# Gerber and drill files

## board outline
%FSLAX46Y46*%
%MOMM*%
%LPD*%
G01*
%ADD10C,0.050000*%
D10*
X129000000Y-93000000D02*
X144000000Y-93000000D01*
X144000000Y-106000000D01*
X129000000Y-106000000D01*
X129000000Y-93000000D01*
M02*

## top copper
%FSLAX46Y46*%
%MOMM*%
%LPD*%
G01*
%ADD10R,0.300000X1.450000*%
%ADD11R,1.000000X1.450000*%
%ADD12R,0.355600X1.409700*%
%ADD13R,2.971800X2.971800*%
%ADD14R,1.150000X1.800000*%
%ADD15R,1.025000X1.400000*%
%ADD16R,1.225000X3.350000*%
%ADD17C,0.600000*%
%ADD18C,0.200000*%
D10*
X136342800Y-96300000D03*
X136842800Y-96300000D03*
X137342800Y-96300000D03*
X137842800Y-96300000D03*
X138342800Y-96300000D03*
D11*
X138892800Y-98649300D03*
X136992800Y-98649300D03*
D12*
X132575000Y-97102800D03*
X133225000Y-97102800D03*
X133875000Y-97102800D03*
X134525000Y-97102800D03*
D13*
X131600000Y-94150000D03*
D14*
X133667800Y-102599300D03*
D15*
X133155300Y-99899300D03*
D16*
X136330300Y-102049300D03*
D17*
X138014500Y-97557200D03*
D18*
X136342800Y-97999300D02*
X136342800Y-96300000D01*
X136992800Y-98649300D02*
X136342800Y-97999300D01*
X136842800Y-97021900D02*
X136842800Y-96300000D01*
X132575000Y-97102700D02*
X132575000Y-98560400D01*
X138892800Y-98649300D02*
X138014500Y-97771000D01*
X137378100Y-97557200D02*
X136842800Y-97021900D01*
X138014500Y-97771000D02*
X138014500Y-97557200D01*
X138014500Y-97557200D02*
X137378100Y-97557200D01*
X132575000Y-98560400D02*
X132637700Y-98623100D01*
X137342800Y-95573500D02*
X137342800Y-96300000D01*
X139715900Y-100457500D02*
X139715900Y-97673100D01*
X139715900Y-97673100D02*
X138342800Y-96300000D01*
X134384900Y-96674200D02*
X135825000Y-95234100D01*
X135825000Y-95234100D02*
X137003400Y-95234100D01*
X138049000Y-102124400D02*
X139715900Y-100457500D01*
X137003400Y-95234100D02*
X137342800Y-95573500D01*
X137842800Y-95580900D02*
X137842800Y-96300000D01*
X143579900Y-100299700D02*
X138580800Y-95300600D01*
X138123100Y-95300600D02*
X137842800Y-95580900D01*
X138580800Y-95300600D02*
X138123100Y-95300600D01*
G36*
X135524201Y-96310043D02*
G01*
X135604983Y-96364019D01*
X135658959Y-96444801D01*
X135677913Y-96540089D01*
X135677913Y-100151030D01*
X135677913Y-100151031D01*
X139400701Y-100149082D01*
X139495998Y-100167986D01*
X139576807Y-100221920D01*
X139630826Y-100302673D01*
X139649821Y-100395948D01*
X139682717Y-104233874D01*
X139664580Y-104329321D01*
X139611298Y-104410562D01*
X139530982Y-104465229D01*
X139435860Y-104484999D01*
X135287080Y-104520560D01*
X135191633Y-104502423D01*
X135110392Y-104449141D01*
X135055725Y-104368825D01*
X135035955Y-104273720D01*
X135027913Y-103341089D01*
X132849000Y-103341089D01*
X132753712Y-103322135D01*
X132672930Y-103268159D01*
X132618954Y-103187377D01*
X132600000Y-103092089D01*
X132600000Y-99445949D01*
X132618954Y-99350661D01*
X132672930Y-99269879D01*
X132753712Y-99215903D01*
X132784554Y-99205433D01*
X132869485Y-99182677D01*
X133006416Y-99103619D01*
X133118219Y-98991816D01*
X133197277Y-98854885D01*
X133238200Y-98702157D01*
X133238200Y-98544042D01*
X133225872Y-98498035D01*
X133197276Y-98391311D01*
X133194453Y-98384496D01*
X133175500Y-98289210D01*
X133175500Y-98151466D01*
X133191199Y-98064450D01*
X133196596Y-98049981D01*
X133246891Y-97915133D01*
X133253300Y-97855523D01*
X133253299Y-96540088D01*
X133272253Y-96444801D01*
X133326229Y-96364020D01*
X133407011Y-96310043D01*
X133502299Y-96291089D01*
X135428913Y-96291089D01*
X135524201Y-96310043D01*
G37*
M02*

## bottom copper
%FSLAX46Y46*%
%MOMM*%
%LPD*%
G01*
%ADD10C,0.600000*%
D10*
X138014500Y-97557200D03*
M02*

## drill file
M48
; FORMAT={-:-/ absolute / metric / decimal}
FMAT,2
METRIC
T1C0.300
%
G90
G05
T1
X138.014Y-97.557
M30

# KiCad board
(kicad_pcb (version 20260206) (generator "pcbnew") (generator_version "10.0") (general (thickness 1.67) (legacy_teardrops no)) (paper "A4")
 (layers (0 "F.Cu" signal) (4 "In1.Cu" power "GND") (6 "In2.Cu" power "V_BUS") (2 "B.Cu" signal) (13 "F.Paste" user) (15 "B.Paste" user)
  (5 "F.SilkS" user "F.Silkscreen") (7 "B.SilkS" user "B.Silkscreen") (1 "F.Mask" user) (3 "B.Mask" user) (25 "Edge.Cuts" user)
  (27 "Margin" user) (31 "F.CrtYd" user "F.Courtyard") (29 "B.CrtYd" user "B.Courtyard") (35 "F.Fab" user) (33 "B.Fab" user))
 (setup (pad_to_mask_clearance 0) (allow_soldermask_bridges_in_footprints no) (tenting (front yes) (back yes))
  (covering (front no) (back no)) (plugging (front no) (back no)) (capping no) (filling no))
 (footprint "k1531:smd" (layer "F.Cu") (at 136.3428 96.3)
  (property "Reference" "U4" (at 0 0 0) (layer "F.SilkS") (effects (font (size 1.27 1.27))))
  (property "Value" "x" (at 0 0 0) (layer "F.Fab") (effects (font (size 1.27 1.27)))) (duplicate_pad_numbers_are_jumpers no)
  (pad "1" smd rect (at 0 0) (size 0.3 1.45) (layers "F.Cu" "F.Mask") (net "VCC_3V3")))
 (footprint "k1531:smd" (layer "F.Cu") (at 136.8428 96.3)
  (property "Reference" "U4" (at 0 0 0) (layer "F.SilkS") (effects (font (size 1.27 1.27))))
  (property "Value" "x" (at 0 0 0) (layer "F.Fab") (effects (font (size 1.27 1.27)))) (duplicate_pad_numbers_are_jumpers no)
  (pad "1" smd rect (at 0 0) (size 0.3 1.45) (layers "F.Cu" "F.Mask") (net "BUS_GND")))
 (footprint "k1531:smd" (layer "F.Cu") (at 137.3428 96.3)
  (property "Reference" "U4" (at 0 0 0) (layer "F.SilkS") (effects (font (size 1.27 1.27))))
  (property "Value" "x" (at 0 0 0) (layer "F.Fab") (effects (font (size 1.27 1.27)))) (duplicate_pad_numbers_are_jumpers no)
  (pad "1" smd rect (at 0 0) (size 0.3 1.45) (layers "F.Cu" "F.Mask") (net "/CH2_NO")))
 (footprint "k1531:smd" (layer "F.Cu") (at 137.8428 96.3)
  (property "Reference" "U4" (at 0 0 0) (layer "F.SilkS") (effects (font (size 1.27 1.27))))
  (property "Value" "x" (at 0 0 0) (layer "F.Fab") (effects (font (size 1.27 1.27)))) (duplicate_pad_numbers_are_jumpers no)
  (pad "1" smd rect (at 0 0) (size 0.3 1.45) (layers "F.Cu" "F.Mask") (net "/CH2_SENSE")))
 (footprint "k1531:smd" (layer "F.Cu") (at 138.3428 96.3)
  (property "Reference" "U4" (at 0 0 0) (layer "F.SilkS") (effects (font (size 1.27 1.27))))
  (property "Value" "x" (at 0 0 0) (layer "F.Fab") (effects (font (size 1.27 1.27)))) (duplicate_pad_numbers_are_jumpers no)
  (pad "1" smd rect (at 0 0) (size 0.3 1.45) (layers "F.Cu" "F.Mask") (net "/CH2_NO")))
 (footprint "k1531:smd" (layer "F.Cu") (at 138.8928 98.6493)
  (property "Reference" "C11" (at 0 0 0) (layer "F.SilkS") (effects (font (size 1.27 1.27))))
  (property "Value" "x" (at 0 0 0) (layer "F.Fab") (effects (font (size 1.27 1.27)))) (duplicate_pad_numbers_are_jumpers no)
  (pad "1" smd rect (at 0 0) (size 1 1.45) (layers "F.Cu" "F.Mask") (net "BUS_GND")))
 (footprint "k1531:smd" (layer "F.Cu") (at 136.9928 98.6493)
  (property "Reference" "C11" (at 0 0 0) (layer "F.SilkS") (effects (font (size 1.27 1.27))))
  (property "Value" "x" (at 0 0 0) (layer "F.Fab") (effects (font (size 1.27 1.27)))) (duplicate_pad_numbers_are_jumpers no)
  (pad "1" smd rect (at 0 0) (size 1 1.45) (layers "F.Cu" "F.Mask") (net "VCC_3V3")))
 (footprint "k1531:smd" (layer "F.Cu") (at 132.575 97.1028)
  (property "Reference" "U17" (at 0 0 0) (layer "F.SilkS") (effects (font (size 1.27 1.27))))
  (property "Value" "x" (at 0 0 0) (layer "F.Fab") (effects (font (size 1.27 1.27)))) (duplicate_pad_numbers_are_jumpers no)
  (pad "1" smd rect (at 0 0) (size 0.3556 1.4097) (layers "F.Cu" "F.Mask") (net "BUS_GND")))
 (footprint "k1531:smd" (layer "F.Cu") (at 133.225 97.1028)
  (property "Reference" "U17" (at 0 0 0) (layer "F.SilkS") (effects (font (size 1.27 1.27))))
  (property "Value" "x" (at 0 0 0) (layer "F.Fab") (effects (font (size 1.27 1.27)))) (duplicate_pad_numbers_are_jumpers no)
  (pad "1" smd rect (at 0 0) (size 0.3556 1.4097) (layers "F.Cu" "F.Mask") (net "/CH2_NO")))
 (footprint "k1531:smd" (layer "F.Cu") (at 133.875 97.1028)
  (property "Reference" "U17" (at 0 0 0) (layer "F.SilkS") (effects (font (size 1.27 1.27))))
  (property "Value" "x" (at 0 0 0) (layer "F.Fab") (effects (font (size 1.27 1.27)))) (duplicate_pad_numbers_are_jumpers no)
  (pad "1" smd rect (at 0 0) (size 0.3556 1.4097) (layers "F.Cu" "F.Mask") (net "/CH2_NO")))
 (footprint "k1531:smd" (layer "F.Cu") (at 134.525 97.1028)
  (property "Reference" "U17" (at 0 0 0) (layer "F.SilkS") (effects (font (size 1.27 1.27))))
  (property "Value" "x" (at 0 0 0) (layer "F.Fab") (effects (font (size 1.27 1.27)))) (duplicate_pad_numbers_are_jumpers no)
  (pad "1" smd rect (at 0 0) (size 0.3556 1.4097) (layers "F.Cu" "F.Mask") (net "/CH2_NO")))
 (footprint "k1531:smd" (layer "F.Cu") (at 131.6 94.15)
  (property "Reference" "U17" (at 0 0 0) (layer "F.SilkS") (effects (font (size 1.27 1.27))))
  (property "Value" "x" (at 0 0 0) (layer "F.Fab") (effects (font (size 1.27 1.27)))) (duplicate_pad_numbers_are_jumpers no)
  (pad "1" smd rect (at 0 0) (size 2.9718 2.9718) (layers "F.Cu" "F.Mask") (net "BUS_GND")))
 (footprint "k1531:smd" (layer "F.Cu") (at 133.6678 102.5993)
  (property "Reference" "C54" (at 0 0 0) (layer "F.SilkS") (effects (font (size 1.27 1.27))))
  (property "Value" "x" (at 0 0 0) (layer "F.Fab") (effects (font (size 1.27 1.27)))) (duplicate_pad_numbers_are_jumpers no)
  (pad "1" smd rect (at 0 0) (size 1.15 1.8) (layers "F.Cu" "F.Mask") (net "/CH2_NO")))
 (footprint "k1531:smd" (layer "F.Cu") (at 133.1553 99.8993)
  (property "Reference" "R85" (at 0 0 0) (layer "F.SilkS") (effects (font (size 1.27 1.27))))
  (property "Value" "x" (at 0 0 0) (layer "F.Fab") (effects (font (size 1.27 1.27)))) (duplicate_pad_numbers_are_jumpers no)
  (pad "1" smd rect (at 0 0) (size 1.025 1.4) (layers "F.Cu" "F.Mask") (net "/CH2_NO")))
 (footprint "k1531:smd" (layer "F.Cu") (at 136.3303 102.0493)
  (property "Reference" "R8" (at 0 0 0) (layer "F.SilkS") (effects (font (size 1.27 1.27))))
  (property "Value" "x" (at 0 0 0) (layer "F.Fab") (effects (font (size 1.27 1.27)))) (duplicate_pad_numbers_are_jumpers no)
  (pad "1" smd rect (at 0 0) (size 1.225 3.35) (layers "F.Cu" "F.Mask") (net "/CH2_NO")))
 (gr_rect (start 129 93) (end 144 106) (stroke (width 0.05) (type default)) (fill no) (layer "Edge.Cuts"))
 (segment (start 136.3428 97.9993) (end 136.3428 96.3) (width 0.2) (layer "F.Cu") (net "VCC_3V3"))
 (segment (start 136.9928 98.6493) (end 136.3428 97.9993) (width 0.2) (layer "F.Cu") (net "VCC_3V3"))
 (segment (start 136.8428 97.0219) (end 136.8428 96.3) (width 0.2) (layer "F.Cu") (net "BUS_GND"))
 (segment (start 132.575 97.1027) (end 132.575 98.5604) (width 0.2) (layer "F.Cu") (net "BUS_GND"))
 (segment (start 138.8928 98.6493) (end 138.0145 97.771) (width 0.2) (layer "F.Cu") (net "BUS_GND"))
 (segment (start 137.3781 97.5572) (end 136.8428 97.0219) (width 0.2) (layer "F.Cu") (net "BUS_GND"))
 (segment (start 138.0145 97.771) (end 138.0145 97.5572) (width 0.2) (layer "F.Cu") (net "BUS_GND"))
 (segment (start 138.0145 97.5572) (end 137.3781 97.5572) (width 0.2) (layer "F.Cu") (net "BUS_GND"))
 (segment (start 132.575 98.5604) (end 132.6377 98.6231) (width 0.2) (layer "F.Cu") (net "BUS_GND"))
 (via (at 138.0145 97.5572) (size 0.6) (drill 0.3) (layers "F.Cu" "B.Cu") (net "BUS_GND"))
 (segment (start 137.3428 95.5735) (end 137.3428 96.3) (width 0.2) (layer "F.Cu") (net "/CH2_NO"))
 (segment (start 139.7159 100.4575) (end 139.7159 97.6731) (width 0.2) (layer "F.Cu") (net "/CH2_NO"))
 (segment (start 139.7159 97.6731) (end 138.3428 96.3) (width 0.2) (layer "F.Cu") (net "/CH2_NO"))
 (segment (start 134.3849 96.6742) (end 135.825 95.2341) (width 0.2) (layer "F.Cu") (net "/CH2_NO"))
 (segment (start 135.825 95.2341) (end 137.0034 95.2341) (width 0.2) (layer "F.Cu") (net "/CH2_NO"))
 (segment (start 138.049 102.1244) (end 139.7159 100.4575) (width 0.2) (layer "F.Cu") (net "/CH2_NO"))
 (segment (start 137.0034 95.2341) (end 137.3428 95.5735) (width 0.2) (layer "F.Cu") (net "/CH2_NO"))
 (segment (start 137.8428 95.5809) (end 137.8428 96.3) (width 0.2) (layer "F.Cu") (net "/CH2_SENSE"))
 (segment (start 143.5799 100.2997) (end 138.5808 95.3006) (width 0.2) (layer "F.Cu") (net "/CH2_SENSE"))
 (segment (start 138.1231 95.3006) (end 137.8428 95.5809) (width 0.2) (layer "F.Cu") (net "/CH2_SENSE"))
 (segment (start 138.5808 95.3006) (end 138.1231 95.3006) (width 0.2) (layer "F.Cu") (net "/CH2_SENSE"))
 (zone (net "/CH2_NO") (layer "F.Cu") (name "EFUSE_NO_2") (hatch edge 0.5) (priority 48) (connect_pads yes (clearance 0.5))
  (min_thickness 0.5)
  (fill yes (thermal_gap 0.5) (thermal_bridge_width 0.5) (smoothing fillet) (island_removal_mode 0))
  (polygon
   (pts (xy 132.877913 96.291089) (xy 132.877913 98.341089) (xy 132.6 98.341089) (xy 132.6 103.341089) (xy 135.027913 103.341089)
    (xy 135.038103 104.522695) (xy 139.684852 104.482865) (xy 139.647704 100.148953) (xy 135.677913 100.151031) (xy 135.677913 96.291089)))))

